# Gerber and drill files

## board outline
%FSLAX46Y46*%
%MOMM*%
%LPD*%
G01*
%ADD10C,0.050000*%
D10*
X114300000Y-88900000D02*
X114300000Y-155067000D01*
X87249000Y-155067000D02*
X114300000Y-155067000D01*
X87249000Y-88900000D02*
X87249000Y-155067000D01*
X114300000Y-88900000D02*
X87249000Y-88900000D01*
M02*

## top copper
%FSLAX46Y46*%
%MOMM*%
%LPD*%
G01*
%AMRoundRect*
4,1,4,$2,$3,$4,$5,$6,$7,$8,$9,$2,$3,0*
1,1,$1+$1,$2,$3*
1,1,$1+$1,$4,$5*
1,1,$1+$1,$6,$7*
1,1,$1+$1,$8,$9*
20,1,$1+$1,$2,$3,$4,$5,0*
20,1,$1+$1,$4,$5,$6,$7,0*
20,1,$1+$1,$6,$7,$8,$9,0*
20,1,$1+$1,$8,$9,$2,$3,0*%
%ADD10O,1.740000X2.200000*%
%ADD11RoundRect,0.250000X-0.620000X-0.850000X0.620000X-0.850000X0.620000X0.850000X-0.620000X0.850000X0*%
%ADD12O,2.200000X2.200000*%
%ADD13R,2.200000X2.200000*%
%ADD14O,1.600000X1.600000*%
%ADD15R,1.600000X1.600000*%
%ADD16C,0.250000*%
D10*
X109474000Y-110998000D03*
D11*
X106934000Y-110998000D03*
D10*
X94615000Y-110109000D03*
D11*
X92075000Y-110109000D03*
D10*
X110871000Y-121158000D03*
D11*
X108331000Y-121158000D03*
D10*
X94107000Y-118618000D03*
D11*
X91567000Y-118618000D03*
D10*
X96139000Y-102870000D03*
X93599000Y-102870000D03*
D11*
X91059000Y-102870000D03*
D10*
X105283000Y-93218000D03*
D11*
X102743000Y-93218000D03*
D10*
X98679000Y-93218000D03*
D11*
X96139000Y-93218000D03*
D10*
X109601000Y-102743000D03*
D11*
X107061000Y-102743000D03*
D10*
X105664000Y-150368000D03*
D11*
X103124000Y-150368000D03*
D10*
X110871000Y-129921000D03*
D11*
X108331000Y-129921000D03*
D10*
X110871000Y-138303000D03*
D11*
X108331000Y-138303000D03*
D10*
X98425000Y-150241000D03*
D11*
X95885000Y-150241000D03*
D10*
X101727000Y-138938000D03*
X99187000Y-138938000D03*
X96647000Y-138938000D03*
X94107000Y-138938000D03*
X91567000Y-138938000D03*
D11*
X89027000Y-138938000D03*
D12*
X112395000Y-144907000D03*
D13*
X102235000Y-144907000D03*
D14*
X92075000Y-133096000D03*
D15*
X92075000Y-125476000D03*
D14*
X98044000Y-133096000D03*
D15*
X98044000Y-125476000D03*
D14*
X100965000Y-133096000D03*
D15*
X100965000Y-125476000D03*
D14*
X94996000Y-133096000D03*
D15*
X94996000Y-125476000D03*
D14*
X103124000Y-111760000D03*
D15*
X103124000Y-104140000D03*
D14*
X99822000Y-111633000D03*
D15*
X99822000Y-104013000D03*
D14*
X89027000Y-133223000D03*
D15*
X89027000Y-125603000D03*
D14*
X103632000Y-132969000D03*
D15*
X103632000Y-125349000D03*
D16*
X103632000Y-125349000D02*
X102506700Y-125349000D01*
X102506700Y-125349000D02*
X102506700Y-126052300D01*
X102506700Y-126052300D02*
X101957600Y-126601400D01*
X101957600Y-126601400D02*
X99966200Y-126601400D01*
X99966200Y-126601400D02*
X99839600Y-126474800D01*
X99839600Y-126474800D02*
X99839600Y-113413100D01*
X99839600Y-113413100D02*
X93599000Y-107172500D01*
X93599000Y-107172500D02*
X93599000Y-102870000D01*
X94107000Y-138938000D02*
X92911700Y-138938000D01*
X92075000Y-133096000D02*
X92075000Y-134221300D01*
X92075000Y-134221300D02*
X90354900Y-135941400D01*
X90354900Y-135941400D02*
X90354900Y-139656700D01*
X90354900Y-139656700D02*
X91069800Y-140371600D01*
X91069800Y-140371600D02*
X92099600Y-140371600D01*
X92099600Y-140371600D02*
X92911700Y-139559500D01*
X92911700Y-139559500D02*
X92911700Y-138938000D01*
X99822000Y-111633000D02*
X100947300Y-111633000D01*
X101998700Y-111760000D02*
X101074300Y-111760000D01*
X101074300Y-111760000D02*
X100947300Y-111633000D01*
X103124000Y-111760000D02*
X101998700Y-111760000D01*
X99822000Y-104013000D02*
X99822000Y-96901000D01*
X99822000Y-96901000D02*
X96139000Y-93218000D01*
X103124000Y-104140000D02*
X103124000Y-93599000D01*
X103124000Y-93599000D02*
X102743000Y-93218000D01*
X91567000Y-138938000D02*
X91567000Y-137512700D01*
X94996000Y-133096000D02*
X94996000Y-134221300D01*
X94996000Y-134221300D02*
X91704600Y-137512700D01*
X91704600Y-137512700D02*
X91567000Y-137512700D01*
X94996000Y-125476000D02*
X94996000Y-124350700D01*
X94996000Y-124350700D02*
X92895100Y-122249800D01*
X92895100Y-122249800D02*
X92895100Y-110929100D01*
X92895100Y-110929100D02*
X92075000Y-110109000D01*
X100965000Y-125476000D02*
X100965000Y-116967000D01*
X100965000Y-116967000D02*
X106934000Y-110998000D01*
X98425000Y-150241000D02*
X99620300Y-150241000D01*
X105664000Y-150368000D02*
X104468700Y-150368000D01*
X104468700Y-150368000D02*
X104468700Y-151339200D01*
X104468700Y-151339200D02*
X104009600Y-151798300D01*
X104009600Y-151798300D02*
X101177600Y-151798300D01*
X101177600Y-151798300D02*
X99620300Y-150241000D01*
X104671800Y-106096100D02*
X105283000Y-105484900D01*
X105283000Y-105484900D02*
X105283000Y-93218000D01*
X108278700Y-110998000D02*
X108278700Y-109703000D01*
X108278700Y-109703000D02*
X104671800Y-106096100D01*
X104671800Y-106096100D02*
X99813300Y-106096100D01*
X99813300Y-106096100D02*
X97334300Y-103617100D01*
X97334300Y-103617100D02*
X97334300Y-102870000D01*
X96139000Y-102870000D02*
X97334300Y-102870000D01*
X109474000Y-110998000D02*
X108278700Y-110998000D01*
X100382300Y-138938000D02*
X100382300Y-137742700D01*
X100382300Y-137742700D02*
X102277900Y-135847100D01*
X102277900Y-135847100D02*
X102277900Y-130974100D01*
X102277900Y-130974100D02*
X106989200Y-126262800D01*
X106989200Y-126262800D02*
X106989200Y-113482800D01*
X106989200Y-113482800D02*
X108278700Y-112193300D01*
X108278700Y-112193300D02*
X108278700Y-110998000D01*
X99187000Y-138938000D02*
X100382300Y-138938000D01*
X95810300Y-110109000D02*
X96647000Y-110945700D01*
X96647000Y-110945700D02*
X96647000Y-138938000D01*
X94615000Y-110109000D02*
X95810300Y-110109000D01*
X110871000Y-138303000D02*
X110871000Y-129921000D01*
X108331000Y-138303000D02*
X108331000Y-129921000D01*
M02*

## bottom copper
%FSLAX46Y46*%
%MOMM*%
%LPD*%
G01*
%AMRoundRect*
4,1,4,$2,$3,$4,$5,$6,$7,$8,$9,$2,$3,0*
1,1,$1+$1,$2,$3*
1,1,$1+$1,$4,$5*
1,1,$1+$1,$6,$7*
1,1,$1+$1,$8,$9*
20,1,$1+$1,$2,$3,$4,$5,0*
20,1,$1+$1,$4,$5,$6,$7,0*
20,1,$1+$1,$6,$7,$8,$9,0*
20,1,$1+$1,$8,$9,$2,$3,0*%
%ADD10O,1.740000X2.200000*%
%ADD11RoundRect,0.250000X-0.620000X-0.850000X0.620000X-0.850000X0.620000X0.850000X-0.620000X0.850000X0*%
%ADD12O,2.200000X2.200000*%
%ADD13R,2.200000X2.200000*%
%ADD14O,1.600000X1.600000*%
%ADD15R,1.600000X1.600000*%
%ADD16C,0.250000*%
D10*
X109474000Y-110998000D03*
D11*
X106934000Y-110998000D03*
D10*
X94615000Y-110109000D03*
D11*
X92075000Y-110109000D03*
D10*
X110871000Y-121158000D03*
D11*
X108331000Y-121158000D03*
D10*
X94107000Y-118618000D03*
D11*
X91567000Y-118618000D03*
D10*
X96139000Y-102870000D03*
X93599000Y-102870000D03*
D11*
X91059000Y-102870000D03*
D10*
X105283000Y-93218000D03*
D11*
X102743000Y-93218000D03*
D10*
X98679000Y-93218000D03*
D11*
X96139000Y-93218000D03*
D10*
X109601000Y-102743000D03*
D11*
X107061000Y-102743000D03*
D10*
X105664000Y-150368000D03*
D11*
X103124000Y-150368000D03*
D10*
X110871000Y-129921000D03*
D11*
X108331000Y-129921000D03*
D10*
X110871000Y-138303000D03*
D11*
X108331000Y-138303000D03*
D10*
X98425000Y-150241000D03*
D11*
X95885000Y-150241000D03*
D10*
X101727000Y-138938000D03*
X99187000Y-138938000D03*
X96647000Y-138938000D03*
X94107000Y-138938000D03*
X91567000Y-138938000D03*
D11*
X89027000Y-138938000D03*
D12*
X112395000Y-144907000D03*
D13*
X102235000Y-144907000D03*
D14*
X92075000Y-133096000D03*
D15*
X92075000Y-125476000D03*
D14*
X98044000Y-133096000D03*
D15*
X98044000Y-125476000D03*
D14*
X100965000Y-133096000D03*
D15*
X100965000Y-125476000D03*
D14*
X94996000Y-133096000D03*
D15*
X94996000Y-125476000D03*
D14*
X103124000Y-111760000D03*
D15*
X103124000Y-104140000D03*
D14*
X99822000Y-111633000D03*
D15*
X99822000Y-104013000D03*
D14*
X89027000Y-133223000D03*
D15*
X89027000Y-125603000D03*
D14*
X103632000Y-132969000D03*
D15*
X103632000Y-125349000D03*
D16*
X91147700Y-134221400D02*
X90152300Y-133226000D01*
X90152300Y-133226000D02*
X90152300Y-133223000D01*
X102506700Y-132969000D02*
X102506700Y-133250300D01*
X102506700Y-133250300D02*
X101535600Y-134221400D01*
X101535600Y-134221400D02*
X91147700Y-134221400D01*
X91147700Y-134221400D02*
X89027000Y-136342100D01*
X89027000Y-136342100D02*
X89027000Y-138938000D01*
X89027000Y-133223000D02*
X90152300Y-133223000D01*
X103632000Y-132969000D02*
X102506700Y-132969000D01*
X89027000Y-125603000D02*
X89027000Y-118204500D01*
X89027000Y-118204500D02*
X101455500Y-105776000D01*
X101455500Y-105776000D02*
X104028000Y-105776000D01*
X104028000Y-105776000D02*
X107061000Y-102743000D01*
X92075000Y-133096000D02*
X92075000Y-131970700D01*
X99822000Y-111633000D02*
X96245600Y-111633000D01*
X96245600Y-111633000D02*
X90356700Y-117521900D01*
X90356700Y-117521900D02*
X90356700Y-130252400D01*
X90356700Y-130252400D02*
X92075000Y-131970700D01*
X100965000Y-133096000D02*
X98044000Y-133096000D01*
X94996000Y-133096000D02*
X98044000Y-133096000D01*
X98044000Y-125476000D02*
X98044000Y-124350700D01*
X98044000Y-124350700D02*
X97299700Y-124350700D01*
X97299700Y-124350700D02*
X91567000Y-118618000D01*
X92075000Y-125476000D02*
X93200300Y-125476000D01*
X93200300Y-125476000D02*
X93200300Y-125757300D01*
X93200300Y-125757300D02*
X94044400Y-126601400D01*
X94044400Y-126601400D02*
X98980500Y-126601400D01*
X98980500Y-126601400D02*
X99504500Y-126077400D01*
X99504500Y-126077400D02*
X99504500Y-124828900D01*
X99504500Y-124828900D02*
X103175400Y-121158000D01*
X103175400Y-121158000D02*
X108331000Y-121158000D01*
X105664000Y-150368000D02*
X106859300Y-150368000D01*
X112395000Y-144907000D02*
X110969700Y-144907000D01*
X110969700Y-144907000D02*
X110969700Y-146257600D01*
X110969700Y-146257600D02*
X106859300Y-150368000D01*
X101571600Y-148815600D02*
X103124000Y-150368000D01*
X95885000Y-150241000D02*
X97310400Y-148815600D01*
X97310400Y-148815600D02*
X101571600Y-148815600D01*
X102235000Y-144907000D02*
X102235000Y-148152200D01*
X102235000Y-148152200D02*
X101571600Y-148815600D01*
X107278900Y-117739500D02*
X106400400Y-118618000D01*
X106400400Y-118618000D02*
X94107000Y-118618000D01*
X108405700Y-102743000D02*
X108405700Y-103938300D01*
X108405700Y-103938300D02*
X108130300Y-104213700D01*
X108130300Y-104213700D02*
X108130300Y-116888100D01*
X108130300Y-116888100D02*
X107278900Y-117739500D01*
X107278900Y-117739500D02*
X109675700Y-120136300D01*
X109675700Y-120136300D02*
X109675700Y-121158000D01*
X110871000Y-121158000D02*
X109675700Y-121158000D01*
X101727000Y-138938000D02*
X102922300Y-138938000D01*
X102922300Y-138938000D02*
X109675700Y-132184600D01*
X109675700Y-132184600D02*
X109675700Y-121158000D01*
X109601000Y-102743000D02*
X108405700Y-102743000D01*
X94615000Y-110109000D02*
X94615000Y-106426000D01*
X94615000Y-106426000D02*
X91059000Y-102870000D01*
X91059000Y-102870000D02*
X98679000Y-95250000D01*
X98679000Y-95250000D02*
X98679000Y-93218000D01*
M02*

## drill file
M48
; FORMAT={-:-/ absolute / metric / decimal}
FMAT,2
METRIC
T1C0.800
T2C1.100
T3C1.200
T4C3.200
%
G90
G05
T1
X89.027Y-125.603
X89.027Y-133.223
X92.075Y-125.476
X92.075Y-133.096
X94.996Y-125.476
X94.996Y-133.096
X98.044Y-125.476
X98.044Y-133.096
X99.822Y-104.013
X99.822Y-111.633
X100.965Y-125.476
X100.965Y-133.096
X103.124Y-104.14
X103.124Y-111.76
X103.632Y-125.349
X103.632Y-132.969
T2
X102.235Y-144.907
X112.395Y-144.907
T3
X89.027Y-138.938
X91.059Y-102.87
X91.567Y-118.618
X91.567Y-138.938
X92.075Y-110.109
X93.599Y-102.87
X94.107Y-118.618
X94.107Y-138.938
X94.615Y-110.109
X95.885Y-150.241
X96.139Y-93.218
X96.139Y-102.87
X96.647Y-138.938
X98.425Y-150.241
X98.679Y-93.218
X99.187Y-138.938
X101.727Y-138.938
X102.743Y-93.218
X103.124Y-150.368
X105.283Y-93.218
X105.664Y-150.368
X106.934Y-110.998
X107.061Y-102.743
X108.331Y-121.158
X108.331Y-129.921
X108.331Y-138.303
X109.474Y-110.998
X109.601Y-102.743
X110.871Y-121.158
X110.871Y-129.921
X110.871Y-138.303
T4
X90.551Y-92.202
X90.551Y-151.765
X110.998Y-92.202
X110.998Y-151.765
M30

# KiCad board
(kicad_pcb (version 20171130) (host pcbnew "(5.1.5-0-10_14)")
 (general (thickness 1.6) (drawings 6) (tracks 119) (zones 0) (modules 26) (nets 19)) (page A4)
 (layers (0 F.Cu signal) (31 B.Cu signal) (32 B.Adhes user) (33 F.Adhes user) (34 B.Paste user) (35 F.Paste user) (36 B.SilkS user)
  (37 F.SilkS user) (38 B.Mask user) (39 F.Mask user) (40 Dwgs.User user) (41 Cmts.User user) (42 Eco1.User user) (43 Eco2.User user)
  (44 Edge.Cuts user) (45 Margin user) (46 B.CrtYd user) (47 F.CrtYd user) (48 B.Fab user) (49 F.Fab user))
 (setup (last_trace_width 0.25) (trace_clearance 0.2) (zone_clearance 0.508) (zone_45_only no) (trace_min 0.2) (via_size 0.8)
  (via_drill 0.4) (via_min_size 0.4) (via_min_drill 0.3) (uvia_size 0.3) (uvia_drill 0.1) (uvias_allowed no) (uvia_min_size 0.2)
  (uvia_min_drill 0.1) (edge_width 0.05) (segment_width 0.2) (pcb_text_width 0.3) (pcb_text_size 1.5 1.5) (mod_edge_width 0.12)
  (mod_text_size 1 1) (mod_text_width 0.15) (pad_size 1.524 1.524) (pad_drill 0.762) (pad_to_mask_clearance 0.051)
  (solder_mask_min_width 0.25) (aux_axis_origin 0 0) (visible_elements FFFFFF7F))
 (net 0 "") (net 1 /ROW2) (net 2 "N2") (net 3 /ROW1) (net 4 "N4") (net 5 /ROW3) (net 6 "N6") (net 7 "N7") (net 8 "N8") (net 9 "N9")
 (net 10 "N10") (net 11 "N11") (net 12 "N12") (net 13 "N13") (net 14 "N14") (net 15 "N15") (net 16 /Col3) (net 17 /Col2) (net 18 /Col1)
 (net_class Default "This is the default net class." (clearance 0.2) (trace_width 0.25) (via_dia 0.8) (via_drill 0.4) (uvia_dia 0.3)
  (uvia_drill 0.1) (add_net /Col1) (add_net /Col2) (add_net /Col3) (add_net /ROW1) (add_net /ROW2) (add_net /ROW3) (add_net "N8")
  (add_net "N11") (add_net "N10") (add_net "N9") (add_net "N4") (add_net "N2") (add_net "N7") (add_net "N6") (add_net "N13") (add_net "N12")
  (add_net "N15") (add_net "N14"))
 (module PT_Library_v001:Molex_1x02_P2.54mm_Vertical (layer F.Cu) (at 106.934 110.998)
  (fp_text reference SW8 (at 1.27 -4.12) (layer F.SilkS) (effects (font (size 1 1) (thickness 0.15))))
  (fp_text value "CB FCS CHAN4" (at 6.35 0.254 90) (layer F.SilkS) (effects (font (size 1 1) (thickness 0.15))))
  (pad 2 thru_hole oval (at 2.54 0) (size 1.74 2.2) (drill 1.2) (layers *.Cu *.Mask) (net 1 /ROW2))
  (pad 1 thru_hole roundrect (at 0 0) (size 1.74 2.2) (drill 1.2) (layers *.Cu *.Mask) (roundrect_rratio 0.143678) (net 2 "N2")))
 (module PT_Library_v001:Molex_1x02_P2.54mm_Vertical (layer F.Cu) (at 92.075 110.109)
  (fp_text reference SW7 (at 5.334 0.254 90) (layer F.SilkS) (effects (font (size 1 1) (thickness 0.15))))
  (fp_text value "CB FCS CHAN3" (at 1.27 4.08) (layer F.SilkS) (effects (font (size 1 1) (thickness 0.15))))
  (pad 2 thru_hole oval (at 2.54 0) (size 1.74 2.2) (drill 1.2) (layers *.Cu *.Mask) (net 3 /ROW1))
  (pad 1 thru_hole roundrect (at 0 0) (size 1.74 2.2) (drill 1.2) (layers *.Cu *.Mask) (roundrect_rratio 0.143678) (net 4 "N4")))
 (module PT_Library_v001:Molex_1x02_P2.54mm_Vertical (layer F.Cu) (at 108.331 121.158)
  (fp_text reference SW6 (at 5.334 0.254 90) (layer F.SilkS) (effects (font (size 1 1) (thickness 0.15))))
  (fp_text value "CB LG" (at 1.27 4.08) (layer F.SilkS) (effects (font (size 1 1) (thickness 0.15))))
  (pad 2 thru_hole oval (at 2.54 0) (size 1.74 2.2) (drill 1.2) (layers *.Cu *.Mask) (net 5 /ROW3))
  (pad 1 thru_hole roundrect (at 0 0) (size 1.74 2.2) (drill 1.2) (layers *.Cu *.Mask) (roundrect_rratio 0.143678) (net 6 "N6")))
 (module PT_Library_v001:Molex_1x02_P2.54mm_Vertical (layer F.Cu) (at 91.567 118.618)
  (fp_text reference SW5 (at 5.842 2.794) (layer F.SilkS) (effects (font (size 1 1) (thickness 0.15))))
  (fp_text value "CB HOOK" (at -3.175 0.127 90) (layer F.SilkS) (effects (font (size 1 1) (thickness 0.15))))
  (pad 2 thru_hole oval (at 2.54 0) (size 1.74 2.2) (drill 1.2) (layers *.Cu *.Mask) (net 5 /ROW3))
  (pad 1 thru_hole roundrect (at 0 0) (size 1.74 2.2) (drill 1.2) (layers *.Cu *.Mask) (roundrect_rratio 0.143678) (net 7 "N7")))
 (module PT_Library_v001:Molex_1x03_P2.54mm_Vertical (layer F.Cu) (at 91.059 102.87)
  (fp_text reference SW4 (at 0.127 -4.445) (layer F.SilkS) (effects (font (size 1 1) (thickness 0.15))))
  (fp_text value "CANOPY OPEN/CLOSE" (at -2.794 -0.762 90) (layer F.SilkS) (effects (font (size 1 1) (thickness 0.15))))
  (pad 3 thru_hole oval (at 5.08 0) (size 1.74 2.2) (drill 1.2) (layers *.Cu *.Mask) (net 1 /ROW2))
  (pad 2 thru_hole oval (at 2.54 0) (size 1.74 2.2) (drill 1.2) (layers *.Cu *.Mask) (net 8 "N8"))
  (pad 1 thru_hole roundrect (at 0 0) (size 1.74 2.2) (drill 1.2) (layers *.Cu *.Mask) (roundrect_rratio 0.143678) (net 3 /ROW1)))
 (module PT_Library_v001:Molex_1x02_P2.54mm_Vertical (layer F.Cu) (at 102.743 93.218)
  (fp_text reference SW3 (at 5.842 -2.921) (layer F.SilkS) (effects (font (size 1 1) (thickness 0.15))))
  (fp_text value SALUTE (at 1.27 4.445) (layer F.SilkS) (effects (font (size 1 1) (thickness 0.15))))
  (pad 2 thru_hole oval (at 2.54 0) (size 1.74 2.2) (drill 1.2) (layers *.Cu *.Mask) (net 1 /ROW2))
  (pad 1 thru_hole roundrect (at 0 0) (size 1.74 2.2) (drill 1.2) (layers *.Cu *.Mask) (roundrect_rratio 0.143678) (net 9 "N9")))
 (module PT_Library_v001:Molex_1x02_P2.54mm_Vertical (layer F.Cu) (at 96.139 93.218)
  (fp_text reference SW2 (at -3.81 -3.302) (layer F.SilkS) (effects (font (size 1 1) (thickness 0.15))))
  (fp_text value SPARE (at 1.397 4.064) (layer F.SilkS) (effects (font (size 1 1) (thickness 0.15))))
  (pad 2 thru_hole oval (at 2.54 0) (size 1.74 2.2) (drill 1.2) (layers *.Cu *.Mask) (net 3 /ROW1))
  (pad 1 thru_hole roundrect (at 0 0) (size 1.74 2.2) (drill 1.2) (layers *.Cu *.Mask) (roundrect_rratio 0.143678) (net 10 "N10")))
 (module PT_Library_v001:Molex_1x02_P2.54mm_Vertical (layer F.Cu) (at 107.061 102.743)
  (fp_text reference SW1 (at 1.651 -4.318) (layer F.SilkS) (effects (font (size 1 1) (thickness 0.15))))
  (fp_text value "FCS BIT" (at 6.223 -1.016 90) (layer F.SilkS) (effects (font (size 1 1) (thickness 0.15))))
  (pad 2 thru_hole oval (at 2.54 0) (size 1.74 2.2) (drill 1.2) (layers *.Cu *.Mask) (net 5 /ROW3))
  (pad 1 thru_hole roundrect (at 0 0) (size 1.74 2.2) (drill 1.2) (layers *.Cu *.Mask) (roundrect_rratio 0.143678) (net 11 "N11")))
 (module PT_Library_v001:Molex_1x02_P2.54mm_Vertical (layer F.Cu) (at 103.124 150.368)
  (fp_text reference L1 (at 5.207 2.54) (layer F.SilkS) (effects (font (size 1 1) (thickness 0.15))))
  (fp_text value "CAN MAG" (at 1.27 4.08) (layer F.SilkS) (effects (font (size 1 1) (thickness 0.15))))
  (pad 2 thru_hole oval (at 2.54 0) (size 1.74 2.2) (drill 1.2) (layers *.Cu *.Mask) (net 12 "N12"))
  (pad 1 thru_hole roundrect (at 0 0) (size 1.74 2.2) (drill 1.2) (layers *.Cu *.Mask) (roundrect_rratio 0.143678) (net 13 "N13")))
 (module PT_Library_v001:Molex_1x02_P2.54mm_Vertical (layer F.Cu) (at 108.331 129.921)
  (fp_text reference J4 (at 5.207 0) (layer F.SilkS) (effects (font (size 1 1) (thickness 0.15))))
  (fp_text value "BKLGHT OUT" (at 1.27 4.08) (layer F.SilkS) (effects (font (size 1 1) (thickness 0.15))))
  (pad 2 thru_hole oval (at 2.54 0) (size 1.74 2.2) (drill 1.2) (layers *.Cu *.Mask) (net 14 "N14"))
  (pad 1 thru_hole roundrect (at 0 0) (size 1.74 2.2) (drill 1.2) (layers *.Cu *.Mask) (roundrect_rratio 0.143678) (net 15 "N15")))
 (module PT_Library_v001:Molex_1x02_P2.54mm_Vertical (layer F.Cu) (at 108.331 138.303)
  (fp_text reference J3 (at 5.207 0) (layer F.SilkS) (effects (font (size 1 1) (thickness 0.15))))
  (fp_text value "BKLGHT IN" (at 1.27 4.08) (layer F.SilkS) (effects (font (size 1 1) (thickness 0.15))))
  (pad 2 thru_hole oval (at 2.54 0) (size 1.74 2.2) (drill 1.2) (layers *.Cu *.Mask) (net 14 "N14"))
  (pad 1 thru_hole roundrect (at 0 0) (size 1.74 2.2) (drill 1.2) (layers *.Cu *.Mask) (roundrect_rratio 0.143678) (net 15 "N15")))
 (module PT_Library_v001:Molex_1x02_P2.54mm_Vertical (layer F.Cu) (at 95.885 150.241)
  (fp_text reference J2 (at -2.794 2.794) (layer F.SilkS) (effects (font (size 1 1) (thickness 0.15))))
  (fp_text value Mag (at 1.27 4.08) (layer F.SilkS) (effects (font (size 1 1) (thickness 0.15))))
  (pad 2 thru_hole oval (at 2.54 0) (size 1.74 2.2) (drill 1.2) (layers *.Cu *.Mask) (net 12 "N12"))
  (pad 1 thru_hole roundrect (at 0 0) (size 1.74 2.2) (drill 1.2) (layers *.Cu *.Mask) (roundrect_rratio 0.143678) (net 13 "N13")))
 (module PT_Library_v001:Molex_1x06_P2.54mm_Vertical (layer F.Cu) (at 89.027 138.938)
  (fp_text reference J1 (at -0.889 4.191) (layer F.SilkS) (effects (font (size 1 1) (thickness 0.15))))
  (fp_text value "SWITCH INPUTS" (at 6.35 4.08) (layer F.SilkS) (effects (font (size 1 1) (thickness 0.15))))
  (pad 6 thru_hole oval (at 12.7 0) (size 1.74 2.2) (drill 1.2) (layers *.Cu *.Mask) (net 5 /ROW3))
  (pad 5 thru_hole oval (at 10.16 0) (size 1.74 2.2) (drill 1.2) (layers *.Cu *.Mask) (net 1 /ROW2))
  (pad 4 thru_hole oval (at 7.62 0) (size 1.74 2.2) (drill 1.2) (layers *.Cu *.Mask) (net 3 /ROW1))
  (pad 3 thru_hole oval (at 5.08 0) (size 1.74 2.2) (drill 1.2) (layers *.Cu *.Mask) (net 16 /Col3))
  (pad 2 thru_hole oval (at 2.54 0) (size 1.74 2.2) (drill 1.2) (layers *.Cu *.Mask) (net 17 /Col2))
  (pad 1 thru_hole roundrect (at 0 0) (size 1.74 2.2) (drill 1.2) (layers *.Cu *.Mask) (roundrect_rratio 0.143678) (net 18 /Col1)))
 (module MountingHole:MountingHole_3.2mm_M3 (layer F.Cu) (at 110.998 151.765)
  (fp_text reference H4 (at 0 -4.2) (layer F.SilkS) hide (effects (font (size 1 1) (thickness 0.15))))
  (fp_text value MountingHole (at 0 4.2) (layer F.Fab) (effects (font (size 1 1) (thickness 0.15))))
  (pad 1 np_thru_hole circle (at 0 0) (size 3.2 3.2) (drill 3.2) (layers *.Cu *.Mask)))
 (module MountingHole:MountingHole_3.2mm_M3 (layer F.Cu) (at 110.998 92.202)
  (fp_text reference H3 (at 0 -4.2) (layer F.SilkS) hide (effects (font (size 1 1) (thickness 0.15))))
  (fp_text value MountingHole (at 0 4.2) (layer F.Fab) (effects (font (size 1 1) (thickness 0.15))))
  (pad 1 np_thru_hole circle (at 0 0) (size 3.2 3.2) (drill 3.2) (layers *.Cu *.Mask)))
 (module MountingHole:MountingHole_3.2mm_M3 (layer F.Cu) (at 90.551 151.765)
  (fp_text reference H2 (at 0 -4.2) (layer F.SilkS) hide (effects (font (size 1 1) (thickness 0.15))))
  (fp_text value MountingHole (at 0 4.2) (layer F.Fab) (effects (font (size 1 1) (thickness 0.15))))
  (pad 1 np_thru_hole circle (at 0 0) (size 3.2 3.2) (drill 3.2) (layers *.Cu *.Mask)))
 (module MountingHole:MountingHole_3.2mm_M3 (layer F.Cu) (at 90.551 92.202)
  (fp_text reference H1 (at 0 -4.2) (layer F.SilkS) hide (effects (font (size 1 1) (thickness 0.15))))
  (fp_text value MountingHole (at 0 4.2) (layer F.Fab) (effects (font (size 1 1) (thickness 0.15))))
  (pad 1 np_thru_hole circle (at 0 0) (size 3.2 3.2) (drill 3.2) (layers *.Cu *.Mask)))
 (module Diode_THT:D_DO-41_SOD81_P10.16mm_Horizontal (layer F.Cu) (at 102.235 144.907)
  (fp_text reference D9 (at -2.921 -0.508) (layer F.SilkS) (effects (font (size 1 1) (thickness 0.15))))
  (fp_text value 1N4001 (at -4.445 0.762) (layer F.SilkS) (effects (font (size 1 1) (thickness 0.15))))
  (pad 2 thru_hole oval (at 10.16 0) (size 2.2 2.2) (drill 1.1) (layers *.Cu *.Mask) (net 12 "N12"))
  (pad 1 thru_hole rect (at 0 0) (size 2.2 2.2) (drill 1.1) (layers *.Cu *.Mask) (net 13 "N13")))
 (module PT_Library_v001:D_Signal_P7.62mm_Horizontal (layer F.Cu) (at 92.075 125.476 270)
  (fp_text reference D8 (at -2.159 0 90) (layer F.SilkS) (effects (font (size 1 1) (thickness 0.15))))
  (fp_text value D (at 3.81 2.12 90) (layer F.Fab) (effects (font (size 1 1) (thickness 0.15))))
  (pad 2 thru_hole oval (at 7.62 0 270) (size 1.6 1.6) (drill 0.8) (layers *.Cu *.Mask) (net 16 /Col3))
  (pad 1 thru_hole rect (at 0 0 270) (size 1.6 1.6) (drill 0.8) (layers *.Cu *.Mask) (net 6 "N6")))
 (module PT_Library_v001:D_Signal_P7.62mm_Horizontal (layer F.Cu) (at 98.044 125.476 270)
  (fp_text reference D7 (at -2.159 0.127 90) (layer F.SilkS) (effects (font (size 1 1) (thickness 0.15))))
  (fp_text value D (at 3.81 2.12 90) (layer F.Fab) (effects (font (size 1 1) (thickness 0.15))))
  (pad 2 thru_hole oval (at 7.62 0 270) (size 1.6 1.6) (drill 0.8) (layers *.Cu *.Mask) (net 17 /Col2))
  (pad 1 thru_hole rect (at 0 0 270) (size 1.6 1.6) (drill 0.8) (layers *.Cu *.Mask) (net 7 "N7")))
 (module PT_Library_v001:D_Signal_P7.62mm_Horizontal (layer F.Cu) (at 100.965 125.476 270)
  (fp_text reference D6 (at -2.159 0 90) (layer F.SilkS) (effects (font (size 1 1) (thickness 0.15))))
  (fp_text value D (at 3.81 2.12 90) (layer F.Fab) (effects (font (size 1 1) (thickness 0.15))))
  (pad 2 thru_hole oval (at 7.62 0 270) (size 1.6 1.6) (drill 0.8) (layers *.Cu *.Mask) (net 17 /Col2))
  (pad 1 thru_hole rect (at 0 0 270) (size 1.6 1.6) (drill 0.8) (layers *.Cu *.Mask) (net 2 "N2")))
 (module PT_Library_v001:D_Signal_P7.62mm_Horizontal (layer F.Cu) (at 94.996 125.476 270)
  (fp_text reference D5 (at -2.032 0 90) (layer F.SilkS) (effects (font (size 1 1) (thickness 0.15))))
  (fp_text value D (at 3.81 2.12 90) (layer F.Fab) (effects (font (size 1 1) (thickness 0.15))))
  (pad 2 thru_hole oval (at 7.62 0 270) (size 1.6 1.6) (drill 0.8) (layers *.Cu *.Mask) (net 17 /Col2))
  (pad 1 thru_hole rect (at 0 0 270) (size 1.6 1.6) (drill 0.8) (layers *.Cu *.Mask) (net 4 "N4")))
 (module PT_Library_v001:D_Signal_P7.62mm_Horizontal (layer F.Cu) (at 103.124 104.14 270)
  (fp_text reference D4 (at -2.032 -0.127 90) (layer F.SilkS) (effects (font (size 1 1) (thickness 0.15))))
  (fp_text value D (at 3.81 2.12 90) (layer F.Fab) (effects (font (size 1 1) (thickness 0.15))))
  (pad 2 thru_hole oval (at 7.62 0 270) (size 1.6 1.6) (drill 0.8) (layers *.Cu *.Mask) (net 16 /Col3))
  (pad 1 thru_hole rect (at 0 0 270) (size 1.6 1.6) (drill 0.8) (layers *.Cu *.Mask) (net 9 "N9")))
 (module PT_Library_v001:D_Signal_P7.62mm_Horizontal (layer F.Cu) (at 99.822 104.013 270)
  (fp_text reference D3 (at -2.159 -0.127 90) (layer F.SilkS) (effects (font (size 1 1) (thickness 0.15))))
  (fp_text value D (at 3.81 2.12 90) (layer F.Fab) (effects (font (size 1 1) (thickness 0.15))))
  (pad 2 thru_hole oval (at 7.62 0 270) (size 1.6 1.6) (drill 0.8) (layers *.Cu *.Mask) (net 16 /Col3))
  (pad 1 thru_hole rect (at 0 0 270) (size 1.6 1.6) (drill 0.8) (layers *.Cu *.Mask) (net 10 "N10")))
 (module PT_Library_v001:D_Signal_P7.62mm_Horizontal (layer F.Cu) (at 89.027 125.603 270)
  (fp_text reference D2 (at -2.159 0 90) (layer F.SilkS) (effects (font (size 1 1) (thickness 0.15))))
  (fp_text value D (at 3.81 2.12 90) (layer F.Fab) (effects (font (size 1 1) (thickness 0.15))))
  (pad 2 thru_hole oval (at 7.62 0 270) (size 1.6 1.6) (drill 0.8) (layers *.Cu *.Mask) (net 18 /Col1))
  (pad 1 thru_hole rect (at 0 0 270) (size 1.6 1.6) (drill 0.8) (layers *.Cu *.Mask) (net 11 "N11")))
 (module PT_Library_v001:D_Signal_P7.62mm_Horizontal (layer F.Cu) (at 103.632 125.349 270)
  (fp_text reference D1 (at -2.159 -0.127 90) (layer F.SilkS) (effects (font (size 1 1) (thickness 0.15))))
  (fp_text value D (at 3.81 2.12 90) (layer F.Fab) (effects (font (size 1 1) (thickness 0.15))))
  (pad 2 thru_hole oval (at 7.62 0 270) (size 1.6 1.6) (drill 0.8) (layers *.Cu *.Mask) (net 18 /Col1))
  (pad 1 thru_hole rect (at 0 0 270) (size 1.6 1.6) (drill 0.8) (layers *.Cu *.Mask) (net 8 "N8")))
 (gr_line (start 114.3 88.9) (end 114.3 155.067) (layer Edge.Cuts) (width 0.05))
 (gr_line (start 87.249 155.067) (end 114.3 155.067) (layer Edge.Cuts) (width 0.05))
 (gr_line (start 87.249 88.9) (end 87.249 155.067) (layer Edge.Cuts) (width 0.05))
 (gr_line (start 114.3 88.9) (end 87.249 88.9) (layer Edge.Cuts) (width 0.05))
 (segment (start 91.1477 134.2214) (end 90.1523 133.226) (width 0.25) (layer B.Cu) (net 18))
 (segment (start 90.1523 133.226) (end 90.1523 133.223) (width 0.25) (layer B.Cu) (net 18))
 (segment (start 102.5067 132.969) (end 102.5067 133.2503) (width 0.25) (layer B.Cu) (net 18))
 (segment (start 102.5067 133.2503) (end 101.5356 134.2214) (width 0.25) (layer B.Cu) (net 18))
 (segment (start 101.5356 134.2214) (end 91.1477 134.2214) (width 0.25) (layer B.Cu) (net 18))
 (segment (start 91.1477 134.2214) (end 89.027 136.3421) (width 0.25) (layer B.Cu) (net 18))
 (segment (start 89.027 136.3421) (end 89.027 138.938) (width 0.25) (layer B.Cu) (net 18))
 (segment (start 89.027 133.223) (end 90.1523 133.223) (width 0.25) (layer B.Cu) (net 18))
 (segment (start 103.632 132.969) (end 102.5067 132.969) (width 0.25) (layer B.Cu) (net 18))
 (segment (start 103.632 125.349) (end 102.5067 125.349) (width 0.25) (layer F.Cu) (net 8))
 (segment (start 102.5067 125.349) (end 102.5067 126.0523) (width 0.25) (layer F.Cu) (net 8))
 (segment (start 102.5067 126.0523) (end 101.9576 126.6014) (width 0.25) (layer F.Cu) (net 8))
 (segment (start 101.9576 126.6014) (end 99.9662 126.6014) (width 0.25) (layer F.Cu) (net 8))
 (segment (start 99.9662 126.6014) (end 99.8396 126.4748) (width 0.25) (layer F.Cu) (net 8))
 (segment (start 99.8396 126.4748) (end 99.8396 113.4131) (width 0.25) (layer F.Cu) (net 8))
 (segment (start 99.8396 113.4131) (end 93.599 107.1725) (width 0.25) (layer F.Cu) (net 8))
 (segment (start 93.599 107.1725) (end 93.599 102.87) (width 0.25) (layer F.Cu) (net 8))
 (segment (start 89.027 125.603) (end 89.027 118.2045) (width 0.25) (layer B.Cu) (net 11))
 (segment (start 89.027 118.2045) (end 101.4555 105.776) (width 0.25) (layer B.Cu) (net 11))
 (segment (start 101.4555 105.776) (end 104.028 105.776) (width 0.25) (layer B.Cu) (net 11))
 (segment (start 104.028 105.776) (end 107.061 102.743) (width 0.25) (layer B.Cu) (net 11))
 (segment (start 92.075 133.096) (end 92.075 131.9707) (width 0.25) (layer B.Cu) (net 16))
 (segment (start 99.822 111.633) (end 96.2456 111.633) (width 0.25) (layer B.Cu) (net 16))
 (segment (start 96.2456 111.633) (end 90.3567 117.5219) (width 0.25) (layer B.Cu) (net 16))
 (segment (start 90.3567 117.5219) (end 90.3567 130.2524) (width 0.25) (layer B.Cu) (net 16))
 (segment (start 90.3567 130.2524) (end 92.075 131.9707) (width 0.25) (layer B.Cu) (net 16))
 (segment (start 94.107 138.938) (end 92.9117 138.938) (width 0.25) (layer F.Cu) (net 16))
 (segment (start 92.075 133.096) (end 92.075 134.2213) (width 0.25) (layer F.Cu) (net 16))
 (segment (start 92.075 134.2213) (end 90.3549 135.9414) (width 0.25) (layer F.Cu) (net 16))
 (segment (start 90.3549 135.9414) (end 90.3549 139.6567) (width 0.25) (layer F.Cu) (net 16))
 (segment (start 90.3549 139.6567) (end 91.0698 140.3716) (width 0.25) (layer F.Cu) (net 16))
 (segment (start 91.0698 140.3716) (end 92.0996 140.3716) (width 0.25) (layer F.Cu) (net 16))
 (segment (start 92.0996 140.3716) (end 92.9117 139.5595) (width 0.25) (layer F.Cu) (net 16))
 (segment (start 92.9117 139.5595) (end 92.9117 138.938) (width 0.25) (layer F.Cu) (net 16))
 (segment (start 99.822 111.633) (end 100.9473 111.633) (width 0.25) (layer F.Cu) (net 16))
 (segment (start 101.9987 111.76) (end 101.0743 111.76) (width 0.25) (layer F.Cu) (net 16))
 (segment (start 101.0743 111.76) (end 100.9473 111.633) (width 0.25) (layer F.Cu) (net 16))
 (segment (start 103.124 111.76) (end 101.9987 111.76) (width 0.25) (layer F.Cu) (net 16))
 (segment (start 99.822 104.013) (end 99.822 96.901) (width 0.25) (layer F.Cu) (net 10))
 (segment (start 99.822 96.901) (end 96.139 93.218) (width 0.25) (layer F.Cu) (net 10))
 (segment (start 103.124 104.14) (end 103.124 93.599) (width 0.25) (layer F.Cu) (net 9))
 (segment (start 103.124 93.599) (end 102.743 93.218) (width 0.25) (layer F.Cu) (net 9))
 (segment (start 91.567 138.938) (end 91.567 137.5127) (width 0.25) (layer F.Cu) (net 17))
 (segment (start 94.996 133.096) (end 94.996 134.2213) (width 0.25) (layer F.Cu) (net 17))
 (segment (start 94.996 134.2213) (end 91.7046 137.5127) (width 0.25) (layer F.Cu) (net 17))
 (segment (start 91.7046 137.5127) (end 91.567 137.5127) (width 0.25) (layer F.Cu) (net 17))
 (segment (start 100.965 133.096) (end 98.044 133.096) (width 0.25) (layer B.Cu) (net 17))
 (segment (start 94.996 133.096) (end 98.044 133.096) (width 0.25) (layer B.Cu) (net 17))
 (segment (start 94.996 125.476) (end 94.996 124.3507) (width 0.25) (layer F.Cu) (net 4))
 (segment (start 94.996 124.3507) (end 92.8951 122.2498) (width 0.25) (layer F.Cu) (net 4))
 (segment (start 92.8951 122.2498) (end 92.8951 110.9291) (width 0.25) (layer F.Cu) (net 4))
 (segment (start 92.8951 110.9291) (end 92.075 110.109) (width 0.25) (layer F.Cu) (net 4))
 (segment (start 100.965 125.476) (end 100.965 116.967) (width 0.25) (layer F.Cu) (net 2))
 (segment (start 100.965 116.967) (end 106.934 110.998) (width 0.25) (layer F.Cu) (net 2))
 (segment (start 98.044 125.476) (end 98.044 124.3507) (width 0.25) (layer B.Cu) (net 7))
 (segment (start 98.044 124.3507) (end 97.2997 124.3507) (width 0.25) (layer B.Cu) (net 7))
 (segment (start 97.2997 124.3507) (end 91.567 118.618) (width 0.25) (layer B.Cu) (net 7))
 (segment (start 92.075 125.476) (end 93.2003 125.476) (width 0.25) (layer B.Cu) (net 6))
 (segment (start 93.2003 125.476) (end 93.2003 125.7573) (width 0.25) (layer B.Cu) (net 6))
 (segment (start 93.2003 125.7573) (end 94.0444 126.6014) (width 0.25) (layer B.Cu) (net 6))
 (segment (start 94.0444 126.6014) (end 98.9805 126.6014) (width 0.25) (layer B.Cu) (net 6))
 (segment (start 98.9805 126.6014) (end 99.5045 126.0774) (width 0.25) (layer B.Cu) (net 6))
 (segment (start 99.5045 126.0774) (end 99.5045 124.8289) (width 0.25) (layer B.Cu) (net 6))
 (segment (start 99.5045 124.8289) (end 103.1754 121.158) (width 0.25) (layer B.Cu) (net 6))
 (segment (start 103.1754 121.158) (end 108.331 121.158) (width 0.25) (layer B.Cu) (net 6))
 (segment (start 98.425 150.241) (end 99.6203 150.241) (width 0.25) (layer F.Cu) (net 12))
 (segment (start 105.664 150.368) (end 104.4687 150.368) (width 0.25) (layer F.Cu) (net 12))
 (segment (start 104.4687 150.368) (end 104.4687 151.3392) (width 0.25) (layer F.Cu) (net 12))
 (segment (start 104.4687 151.3392) (end 104.0096 151.7983) (width 0.25) (layer F.Cu) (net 12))
 (segment (start 104.0096 151.7983) (end 101.1776 151.7983) (width 0.25) (layer F.Cu) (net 12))
 (segment (start 101.1776 151.7983) (end 99.6203 150.241) (width 0.25) (layer F.Cu) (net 12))
 (segment (start 105.664 150.368) (end 106.8593 150.368) (width 0.25) (layer B.Cu) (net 12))
 (segment (start 112.395 144.907) (end 110.9697 144.907) (width 0.25) (layer B.Cu) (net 12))
 (segment (start 110.9697 144.907) (end 110.9697 146.2576) (width 0.25) (layer B.Cu) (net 12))
 (segment (start 110.9697 146.2576) (end 106.8593 150.368) (width 0.25) (layer B.Cu) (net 12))
 (segment (start 101.5716 148.8156) (end 103.124 150.368) (width 0.25) (layer B.Cu) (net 13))
 (segment (start 95.885 150.241) (end 97.3104 148.8156) (width 0.25) (layer B.Cu) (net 13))
 (segment (start 97.3104 148.8156) (end 101.5716 148.8156) (width 0.25) (layer B.Cu) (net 13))
 (segment (start 102.235 144.907) (end 102.235 148.1522) (width 0.25) (layer B.Cu) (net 13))
 (segment (start 102.235 148.1522) (end 101.5716 148.8156) (width 0.25) (layer B.Cu) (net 13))
 (segment (start 107.2789 117.7395) (end 106.4004 118.618) (width 0.25) (layer B.Cu) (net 5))
 (segment (start 106.4004 118.618) (end 94.107 118.618) (width 0.25) (layer B.Cu) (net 5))
 (segment (start 108.4057 102.743) (end 108.4057 103.9383) (width 0.25) (layer B.Cu) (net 5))
 (segment (start 108.4057 103.9383) (end 108.1303 104.2137) (width 0.25) (layer B.Cu) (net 5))
 (segment (start 108.1303 104.2137) (end 108.1303 116.8881) (width 0.25) (layer B.Cu) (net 5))
 (segment (start 108.1303 116.8881) (end 107.2789 117.7395) (width 0.25) (layer B.Cu) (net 5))
 (segment (start 107.2789 117.7395) (end 109.6757 120.1363) (width 0.25) (layer B.Cu) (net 5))
 (segment (start 109.6757 120.1363) (end 109.6757 121.158) (width 0.25) (layer B.Cu) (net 5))
 (segment (start 110.871 121.158) (end 109.6757 121.158) (width 0.25) (layer B.Cu) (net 5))
 (segment (start 101.727 138.938) (end 102.9223 138.938) (width 0.25) (layer B.Cu) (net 5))
 (segment (start 102.9223 138.938) (end 109.6757 132.1846) (width 0.25) (layer B.Cu) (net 5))
 (segment (start 109.6757 132.1846) (end 109.6757 121.158) (width 0.25) (layer B.Cu) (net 5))
 (segment (start 109.601 102.743) (end 108.4057 102.743) (width 0.25) (layer B.Cu) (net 5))
 (segment (start 104.6718 106.0961) (end 105.283 105.4849) (width 0.25) (layer F.Cu) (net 1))
 (segment (start 105.283 105.4849) (end 105.283 93.218) (width 0.25) (layer F.Cu) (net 1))
 (segment (start 108.2787 110.998) (end 108.2787 109.703) (width 0.25) (layer F.Cu) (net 1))
 (segment (start 108.2787 109.703) (end 104.6718 106.0961) (width 0.25) (layer F.Cu) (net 1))
 (segment (start 104.6718 106.0961) (end 99.8133 106.0961) (width 0.25) (layer F.Cu) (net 1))
 (segment (start 99.8133 106.0961) (end 97.3343 103.6171) (width 0.25) (layer F.Cu) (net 1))
 (segment (start 97.3343 103.6171) (end 97.3343 102.87) (width 0.25) (layer F.Cu) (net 1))
 (segment (start 96.139 102.87) (end 97.3343 102.87) (width 0.25) (layer F.Cu) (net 1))
 (segment (start 109.474 110.998) (end 108.2787 110.998) (width 0.25) (layer F.Cu) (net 1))
 (segment (start 100.3823 138.938) (end 100.3823 137.7427) (width 0.25) (layer F.Cu) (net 1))
 (segment (start 100.3823 137.7427) (end 102.2779 135.8471) (width 0.25) (layer F.Cu) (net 1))
 (segment (start 102.2779 135.8471) (end 102.2779 130.9741) (width 0.25) (layer F.Cu) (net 1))
 (segment (start 102.2779 130.9741) (end 106.9892 126.2628) (width 0.25) (layer F.Cu) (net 1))
 (segment (start 106.9892 126.2628) (end 106.9892 113.4828) (width 0.25) (layer F.Cu) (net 1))
 (segment (start 106.9892 113.4828) (end 108.2787 112.1933) (width 0.25) (layer F.Cu) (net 1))
 (segment (start 108.2787 112.1933) (end 108.2787 110.998) (width 0.25) (layer F.Cu) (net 1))
 (segment (start 99.187 138.938) (end 100.3823 138.938) (width 0.25) (layer F.Cu) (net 1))
 (segment (start 95.8103 110.109) (end 96.647 110.9457) (width 0.25) (layer F.Cu) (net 3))
 (segment (start 96.647 110.9457) (end 96.647 138.938) (width 0.25) (layer F.Cu) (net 3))
 (segment (start 94.615 110.109) (end 94.615 106.426) (width 0.25) (layer B.Cu) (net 3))
 (segment (start 94.615 106.426) (end 91.059 102.87) (width 0.25) (layer B.Cu) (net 3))
 (segment (start 91.059 102.87) (end 98.679 95.25) (width 0.25) (layer B.Cu) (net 3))
 (segment (start 98.679 95.25) (end 98.679 93.218) (width 0.25) (layer B.Cu) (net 3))
 (segment (start 94.615 110.109) (end 95.8103 110.109) (width 0.25) (layer F.Cu) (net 3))
 (segment (start 110.871 138.303) (end 110.871 129.921) (width 0.25) (layer F.Cu) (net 14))
 (segment (start 108.331 138.303) (end 108.331 129.921) (width 0.25) (layer F.Cu) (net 15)))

